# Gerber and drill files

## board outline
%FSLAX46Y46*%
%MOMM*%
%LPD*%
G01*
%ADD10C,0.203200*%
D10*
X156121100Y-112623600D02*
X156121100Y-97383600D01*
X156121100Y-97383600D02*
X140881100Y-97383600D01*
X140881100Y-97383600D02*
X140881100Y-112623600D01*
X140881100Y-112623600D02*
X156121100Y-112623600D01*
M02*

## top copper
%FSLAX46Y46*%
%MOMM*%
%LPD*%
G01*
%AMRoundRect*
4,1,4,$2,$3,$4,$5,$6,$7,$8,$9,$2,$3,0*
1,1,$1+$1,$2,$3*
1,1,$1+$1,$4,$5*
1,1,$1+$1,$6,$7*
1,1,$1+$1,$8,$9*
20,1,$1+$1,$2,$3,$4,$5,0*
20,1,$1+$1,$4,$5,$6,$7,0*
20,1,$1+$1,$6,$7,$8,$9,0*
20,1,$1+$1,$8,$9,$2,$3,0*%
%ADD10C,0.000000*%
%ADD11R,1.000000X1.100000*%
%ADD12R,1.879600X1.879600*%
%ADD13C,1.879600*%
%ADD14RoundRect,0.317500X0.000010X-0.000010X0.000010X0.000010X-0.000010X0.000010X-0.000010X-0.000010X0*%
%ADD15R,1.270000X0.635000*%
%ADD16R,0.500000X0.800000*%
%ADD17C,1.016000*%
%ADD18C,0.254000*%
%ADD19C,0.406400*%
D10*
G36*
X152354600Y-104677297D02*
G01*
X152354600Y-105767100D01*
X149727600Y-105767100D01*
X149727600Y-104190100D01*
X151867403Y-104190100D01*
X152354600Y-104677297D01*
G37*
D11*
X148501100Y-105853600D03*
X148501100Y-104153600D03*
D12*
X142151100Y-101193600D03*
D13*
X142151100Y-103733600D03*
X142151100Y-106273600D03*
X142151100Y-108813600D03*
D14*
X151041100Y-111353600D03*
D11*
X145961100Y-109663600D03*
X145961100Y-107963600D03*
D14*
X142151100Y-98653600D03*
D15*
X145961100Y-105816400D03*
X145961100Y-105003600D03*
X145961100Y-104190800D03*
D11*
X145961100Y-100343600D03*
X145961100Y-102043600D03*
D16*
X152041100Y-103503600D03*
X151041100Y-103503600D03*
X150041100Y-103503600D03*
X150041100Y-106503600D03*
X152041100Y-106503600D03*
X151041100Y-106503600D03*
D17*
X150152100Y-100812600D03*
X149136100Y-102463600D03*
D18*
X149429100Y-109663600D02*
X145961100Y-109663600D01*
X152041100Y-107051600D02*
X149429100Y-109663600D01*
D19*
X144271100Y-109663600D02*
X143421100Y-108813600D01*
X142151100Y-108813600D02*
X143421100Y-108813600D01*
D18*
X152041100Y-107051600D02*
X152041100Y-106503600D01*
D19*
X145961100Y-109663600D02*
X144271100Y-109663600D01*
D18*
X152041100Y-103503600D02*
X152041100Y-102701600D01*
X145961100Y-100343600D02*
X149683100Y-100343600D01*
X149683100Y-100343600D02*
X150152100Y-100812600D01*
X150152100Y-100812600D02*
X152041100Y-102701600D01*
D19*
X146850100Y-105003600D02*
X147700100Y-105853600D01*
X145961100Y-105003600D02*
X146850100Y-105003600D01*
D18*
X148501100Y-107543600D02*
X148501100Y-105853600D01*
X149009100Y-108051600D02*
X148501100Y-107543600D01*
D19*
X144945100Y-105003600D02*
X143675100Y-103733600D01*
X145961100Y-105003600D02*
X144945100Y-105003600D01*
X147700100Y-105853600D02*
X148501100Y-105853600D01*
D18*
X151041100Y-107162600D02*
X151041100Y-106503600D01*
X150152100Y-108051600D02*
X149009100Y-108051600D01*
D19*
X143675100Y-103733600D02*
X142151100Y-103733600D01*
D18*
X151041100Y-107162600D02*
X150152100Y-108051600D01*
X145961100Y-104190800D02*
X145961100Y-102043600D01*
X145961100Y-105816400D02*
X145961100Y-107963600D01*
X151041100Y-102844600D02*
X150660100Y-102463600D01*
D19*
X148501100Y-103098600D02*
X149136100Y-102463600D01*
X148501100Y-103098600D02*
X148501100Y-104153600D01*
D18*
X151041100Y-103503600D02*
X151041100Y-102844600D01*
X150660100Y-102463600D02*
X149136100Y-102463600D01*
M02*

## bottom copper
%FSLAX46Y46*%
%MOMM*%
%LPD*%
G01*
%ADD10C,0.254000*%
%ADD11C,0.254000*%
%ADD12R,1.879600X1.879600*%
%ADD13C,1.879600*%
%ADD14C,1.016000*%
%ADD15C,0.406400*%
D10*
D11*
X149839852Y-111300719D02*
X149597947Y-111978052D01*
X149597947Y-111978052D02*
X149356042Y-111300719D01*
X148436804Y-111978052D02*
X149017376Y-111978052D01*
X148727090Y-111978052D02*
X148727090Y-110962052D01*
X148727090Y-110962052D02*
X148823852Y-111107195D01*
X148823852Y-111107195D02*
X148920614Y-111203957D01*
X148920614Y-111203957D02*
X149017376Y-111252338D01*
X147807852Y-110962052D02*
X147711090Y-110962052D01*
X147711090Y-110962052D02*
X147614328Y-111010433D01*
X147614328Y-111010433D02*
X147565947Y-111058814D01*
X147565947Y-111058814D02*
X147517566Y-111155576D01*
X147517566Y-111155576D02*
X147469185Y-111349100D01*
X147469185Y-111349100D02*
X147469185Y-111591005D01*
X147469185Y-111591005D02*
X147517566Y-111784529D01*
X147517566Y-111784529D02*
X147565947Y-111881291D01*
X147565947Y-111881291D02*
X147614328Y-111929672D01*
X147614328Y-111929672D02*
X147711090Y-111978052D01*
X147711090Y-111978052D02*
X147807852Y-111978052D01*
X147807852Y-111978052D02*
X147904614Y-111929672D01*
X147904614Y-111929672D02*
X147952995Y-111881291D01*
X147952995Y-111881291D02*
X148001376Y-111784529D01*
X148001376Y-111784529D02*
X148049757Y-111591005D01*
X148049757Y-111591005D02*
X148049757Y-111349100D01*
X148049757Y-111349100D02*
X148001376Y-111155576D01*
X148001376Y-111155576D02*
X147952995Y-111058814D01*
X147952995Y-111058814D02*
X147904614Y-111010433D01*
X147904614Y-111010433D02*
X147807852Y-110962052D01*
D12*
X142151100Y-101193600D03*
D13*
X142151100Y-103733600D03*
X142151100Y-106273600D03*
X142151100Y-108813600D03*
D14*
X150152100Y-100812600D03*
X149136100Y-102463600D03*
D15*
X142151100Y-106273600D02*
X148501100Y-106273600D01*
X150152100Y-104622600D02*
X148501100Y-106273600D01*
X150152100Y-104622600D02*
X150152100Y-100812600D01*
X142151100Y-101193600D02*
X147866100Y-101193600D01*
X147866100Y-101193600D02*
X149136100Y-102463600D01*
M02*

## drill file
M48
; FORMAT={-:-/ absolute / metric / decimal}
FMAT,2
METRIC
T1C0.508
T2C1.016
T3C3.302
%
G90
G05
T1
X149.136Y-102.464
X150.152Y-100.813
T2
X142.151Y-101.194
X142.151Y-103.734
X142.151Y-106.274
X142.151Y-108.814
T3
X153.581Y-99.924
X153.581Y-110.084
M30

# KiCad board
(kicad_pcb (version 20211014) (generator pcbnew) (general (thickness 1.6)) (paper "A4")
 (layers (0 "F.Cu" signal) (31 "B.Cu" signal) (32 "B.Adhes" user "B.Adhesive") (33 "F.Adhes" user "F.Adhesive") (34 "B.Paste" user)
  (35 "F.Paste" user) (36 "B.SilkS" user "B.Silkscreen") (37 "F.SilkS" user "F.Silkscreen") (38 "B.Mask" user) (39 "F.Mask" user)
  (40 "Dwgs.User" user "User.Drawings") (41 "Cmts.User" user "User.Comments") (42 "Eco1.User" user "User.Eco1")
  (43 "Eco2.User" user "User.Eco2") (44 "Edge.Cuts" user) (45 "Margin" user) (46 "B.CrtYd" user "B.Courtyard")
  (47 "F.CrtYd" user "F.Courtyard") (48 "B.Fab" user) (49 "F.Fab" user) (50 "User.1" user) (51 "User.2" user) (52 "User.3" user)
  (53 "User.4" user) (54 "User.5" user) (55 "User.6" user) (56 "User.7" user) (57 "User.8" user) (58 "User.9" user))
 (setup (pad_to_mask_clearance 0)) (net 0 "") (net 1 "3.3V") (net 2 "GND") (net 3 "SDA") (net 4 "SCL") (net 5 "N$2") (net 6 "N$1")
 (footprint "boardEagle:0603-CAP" (layer "F.Cu") (at 148.5011 105.0036 90)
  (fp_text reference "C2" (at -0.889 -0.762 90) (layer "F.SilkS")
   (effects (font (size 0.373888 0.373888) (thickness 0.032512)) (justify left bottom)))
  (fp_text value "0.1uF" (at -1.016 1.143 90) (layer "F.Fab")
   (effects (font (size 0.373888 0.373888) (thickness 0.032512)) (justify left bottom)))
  (pad "1" smd rect (at -0.85 0 90) (size 1.1 1) (layers "F.Cu" "F.Paste" "F.Mask") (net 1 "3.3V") (solder_mask_margin 0.1016))
  (pad "2" smd rect (at 0.85 0 90) (size 1.1 1) (layers "F.Cu" "F.Paste" "F.Mask") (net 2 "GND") (solder_mask_margin 0.1016)))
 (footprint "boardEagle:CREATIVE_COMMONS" (layer "F.Cu") (at 128.1811 121.5136)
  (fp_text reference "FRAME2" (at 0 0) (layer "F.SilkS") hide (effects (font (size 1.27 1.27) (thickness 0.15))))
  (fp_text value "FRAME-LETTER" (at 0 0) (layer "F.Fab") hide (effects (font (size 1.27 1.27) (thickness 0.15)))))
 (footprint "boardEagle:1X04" (layer "F.Cu") (at 142.1511 101.1936 -90)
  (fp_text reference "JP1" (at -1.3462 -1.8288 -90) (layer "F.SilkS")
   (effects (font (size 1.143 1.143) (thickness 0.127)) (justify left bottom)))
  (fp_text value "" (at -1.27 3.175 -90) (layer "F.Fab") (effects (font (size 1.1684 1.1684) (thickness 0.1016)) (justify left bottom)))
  (pad "1" thru_hole rect (at 0 0) (size 1.8796 1.8796) (drill 1.016) (layers *.Cu *.Mask) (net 2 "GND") (solder_mask_margin 0.1016))
  (pad "2" thru_hole circle (at 2.54 0) (size 1.8796 1.8796) (drill 1.016) (layers *.Cu *.Mask) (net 1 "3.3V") (solder_mask_margin 0.1016))
  (pad "3" thru_hole circle (at 5.08 0) (size 1.8796 1.8796) (drill 1.016) (layers *.Cu *.Mask) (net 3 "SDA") (solder_mask_margin 0.1016))
  (pad "4" thru_hole circle (at 7.62 0) (size 1.8796 1.8796) (drill 1.016) (layers *.Cu *.Mask) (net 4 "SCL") (solder_mask_margin 0.1016)))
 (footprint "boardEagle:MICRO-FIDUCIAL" (layer "F.Cu") (at 151.0411 111.3536 90)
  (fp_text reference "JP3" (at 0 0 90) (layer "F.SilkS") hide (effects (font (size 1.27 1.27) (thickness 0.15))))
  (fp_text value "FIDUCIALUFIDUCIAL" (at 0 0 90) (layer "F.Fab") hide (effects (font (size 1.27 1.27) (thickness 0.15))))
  (pad "1" smd roundrect (at 0 0 90) (size 0.635 0.635) (layers "F.Cu" "F.Mask") (roundrect_rratio 0.5) (solder_mask_margin 0.1016)))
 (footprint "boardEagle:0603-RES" (layer "F.Cu") (at 145.9611 108.8136 90)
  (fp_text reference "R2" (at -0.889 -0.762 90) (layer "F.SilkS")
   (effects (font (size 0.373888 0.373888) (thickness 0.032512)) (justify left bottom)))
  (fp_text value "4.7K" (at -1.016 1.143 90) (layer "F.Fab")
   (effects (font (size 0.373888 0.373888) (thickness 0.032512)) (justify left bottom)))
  (pad "1" smd rect (at -0.85 0 90) (size 1.1 1) (layers "F.Cu" "F.Paste" "F.Mask") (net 4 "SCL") (solder_mask_margin 0.1016))
  (pad "2" smd rect (at 0.85 0 90) (size 1.1 1) (layers "F.Cu" "F.Paste" "F.Mask") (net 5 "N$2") (solder_mask_margin 0.1016)))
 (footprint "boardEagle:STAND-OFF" (layer "F.Cu") (at 153.5811 99.9236 90)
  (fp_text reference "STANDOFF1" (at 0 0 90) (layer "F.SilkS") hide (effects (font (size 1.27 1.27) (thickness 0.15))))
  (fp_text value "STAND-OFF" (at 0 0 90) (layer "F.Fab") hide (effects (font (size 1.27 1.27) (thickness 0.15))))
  (pad "" np_thru_hole circle (at 0 0 90) (size 3.302 3.302) (drill 3.302) (layers *.Cu *.Mask)))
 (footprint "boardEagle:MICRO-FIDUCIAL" (layer "F.Cu") (at 142.1511 98.6536 90)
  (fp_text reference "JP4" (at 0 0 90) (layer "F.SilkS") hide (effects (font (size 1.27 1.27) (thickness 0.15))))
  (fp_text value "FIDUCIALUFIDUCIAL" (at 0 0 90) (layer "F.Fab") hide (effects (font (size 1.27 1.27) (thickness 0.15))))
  (pad "1" smd roundrect (at 0 0 90) (size 0.635 0.635) (layers "F.Cu" "F.Mask") (roundrect_rratio 0.5) (solder_mask_margin 0.1016)))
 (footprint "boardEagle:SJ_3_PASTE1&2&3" (layer "F.Cu") (at 145.9611 105.0036 90)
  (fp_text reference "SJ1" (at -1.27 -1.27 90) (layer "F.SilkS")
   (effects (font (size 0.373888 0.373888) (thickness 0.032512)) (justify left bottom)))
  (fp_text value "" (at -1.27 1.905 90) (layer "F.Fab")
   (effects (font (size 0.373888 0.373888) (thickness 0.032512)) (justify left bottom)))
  (pad "1" smd rect (at -0.8128 0 90) (size 0.635 1.27) (layers "F.Cu" "F.Mask") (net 5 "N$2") (solder_mask_margin 0.1016))
  (pad "2" smd rect (at 0 0 90) (size 0.635 1.27) (layers "F.Cu" "F.Mask") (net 1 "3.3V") (solder_mask_margin 0.1016))
  (pad "3" smd rect (at 0.8128 0 90) (size 0.635 1.27) (layers "F.Cu" "F.Mask") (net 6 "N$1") (solder_mask_margin 0.1016)))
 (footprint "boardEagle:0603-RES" (layer "F.Cu") (at 145.9611 101.1936 -90)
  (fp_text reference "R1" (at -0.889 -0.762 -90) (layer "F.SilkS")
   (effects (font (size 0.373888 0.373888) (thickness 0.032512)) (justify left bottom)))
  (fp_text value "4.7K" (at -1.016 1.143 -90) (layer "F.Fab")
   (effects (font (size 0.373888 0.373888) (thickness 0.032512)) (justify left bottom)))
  (pad "1" smd rect (at -0.85 0 270) (size 1.1 1) (layers "F.Cu" "F.Paste" "F.Mask") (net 3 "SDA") (solder_mask_margin 0.1016))
  (pad "2" smd rect (at 0.85 0 270) (size 1.1 1) (layers "F.Cu" "F.Paste" "F.Mask") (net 6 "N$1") (solder_mask_margin 0.1016)))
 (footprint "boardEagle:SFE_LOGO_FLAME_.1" (layer "F.Cu") (at 152.9461 106.4006)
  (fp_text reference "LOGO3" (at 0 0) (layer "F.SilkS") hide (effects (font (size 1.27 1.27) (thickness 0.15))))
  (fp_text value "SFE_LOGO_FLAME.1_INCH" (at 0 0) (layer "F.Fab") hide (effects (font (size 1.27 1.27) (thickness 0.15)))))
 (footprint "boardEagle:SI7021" (layer "F.Cu") (at 151.0411 105.0036 90)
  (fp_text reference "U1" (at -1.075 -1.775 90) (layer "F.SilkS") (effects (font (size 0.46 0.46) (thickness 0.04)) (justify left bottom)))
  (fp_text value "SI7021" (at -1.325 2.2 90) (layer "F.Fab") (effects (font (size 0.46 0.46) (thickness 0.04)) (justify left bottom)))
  (fp_poly
   (pts (xy 0.8135 0.826303) (xy 0.326303 1.3135) (xy -0.7635 1.3135) (xy -0.7635 -1.3135) (xy 0.8135 -1.3135)) (layer "F.Cu") (width 0)
   (fill solid))
  (pad "DATA" smd rect (at 1.5 1) (size 0.5 0.8) (layers "F.Cu" "F.Paste" "F.Mask") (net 3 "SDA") (solder_mask_margin 0.1016))
  (pad "GND" smd rect (at 1.5 0) (size 0.5 0.8) (layers "F.Cu" "F.Paste" "F.Mask") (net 2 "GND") (solder_mask_margin 0.1016))
  (pad "NC@3" smd rect (at 1.5 -1) (size 0.5 0.8) (layers "F.Cu" "F.Paste" "F.Mask") (solder_mask_margin 0.1016))
  (pad "NC@4" smd rect (at -1.5 -1) (size 0.5 0.8) (layers "F.Cu" "F.Paste" "F.Mask") (solder_mask_margin 0.1016))
  (pad "SCK" smd rect (at -1.5 1) (size 0.5 0.8) (layers "F.Cu" "F.Paste" "F.Mask") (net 4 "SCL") (solder_mask_margin 0.1016))
  (pad "VDD" smd rect (at -1.5 0) (size 0.5 0.8) (layers "F.Cu" "F.Paste" "F.Mask") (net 1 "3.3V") (solder_mask_margin 0.1016)))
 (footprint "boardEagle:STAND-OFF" (layer "F.Cu") (at 153.5811 110.0836 90)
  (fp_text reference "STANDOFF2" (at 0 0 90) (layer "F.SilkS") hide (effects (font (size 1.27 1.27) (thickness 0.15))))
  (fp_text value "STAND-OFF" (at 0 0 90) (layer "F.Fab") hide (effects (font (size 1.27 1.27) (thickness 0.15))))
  (pad "" np_thru_hole circle (at 0 0 90) (size 3.302 3.302) (drill 3.302) (layers *.Cu *.Mask)))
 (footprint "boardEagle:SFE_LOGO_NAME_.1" (layer "B.Cu") (at 149.7711 98.6536 -90)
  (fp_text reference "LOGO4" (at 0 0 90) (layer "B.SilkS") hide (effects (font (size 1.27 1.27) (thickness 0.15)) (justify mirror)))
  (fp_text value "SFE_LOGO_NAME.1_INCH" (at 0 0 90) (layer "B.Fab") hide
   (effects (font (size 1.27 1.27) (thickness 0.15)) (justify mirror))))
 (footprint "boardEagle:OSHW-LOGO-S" (layer "B.Cu") (at 153.5811 105.1306 -90)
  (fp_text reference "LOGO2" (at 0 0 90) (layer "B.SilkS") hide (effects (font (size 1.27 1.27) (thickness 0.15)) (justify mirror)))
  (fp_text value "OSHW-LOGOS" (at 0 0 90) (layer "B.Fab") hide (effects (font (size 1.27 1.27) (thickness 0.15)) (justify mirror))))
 (gr_line (start 156.1211 112.6236) (end 156.1211 97.3836) (layer "Edge.Cuts") (width 0.2032))
 (gr_line (start 156.1211 97.3836) (end 140.8811 97.3836) (layer "Edge.Cuts") (width 0.2032))
 (gr_line (start 140.8811 97.3836) (end 140.8811 112.6236) (layer "Edge.Cuts") (width 0.2032))
 (gr_line (start 140.8811 112.6236) (end 156.1211 112.6236) (layer "Edge.Cuts") (width 0.2032))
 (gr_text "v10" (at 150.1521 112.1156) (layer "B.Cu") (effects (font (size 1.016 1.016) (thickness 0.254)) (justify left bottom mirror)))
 (segment (start 149.4291 109.6636) (end 145.9611 109.6636) (width 0.254) (layer "F.Cu") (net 4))
 (segment (start 152.0411 107.0516) (end 149.4291 109.6636) (width 0.254) (layer "F.Cu") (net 4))
 (segment (start 144.2711 109.6636) (end 143.4211 108.8136) (width 0.4064) (layer "F.Cu") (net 4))
 (segment (start 142.1511 108.8136) (end 143.4211 108.8136) (width 0.4064) (layer "F.Cu") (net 4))
 (segment (start 152.0411 107.0516) (end 152.0411 106.5036) (width 0.254) (layer "F.Cu") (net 4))
 (segment (start 145.9611 109.6636) (end 144.2711 109.6636) (width 0.4064) (layer "F.Cu") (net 4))
 (segment (start 152.0411 103.5036) (end 152.0411 102.7016) (width 0.254) (layer "F.Cu") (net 3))
 (segment (start 145.9611 100.3436) (end 149.6831 100.3436) (width 0.254) (layer "F.Cu") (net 3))
 (segment (start 149.6831 100.3436) (end 150.1521 100.8126) (width 0.254) (layer "F.Cu") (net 3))
 (segment (start 150.1521 100.8126) (end 152.0411 102.7016) (width 0.254) (layer "F.Cu") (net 3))
 (via (at 150.1521 100.8126) (size 1.016) (drill 0.508) (layers "F.Cu" "B.Cu") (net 3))
 (segment (start 142.1511 106.2736) (end 148.5011 106.2736) (width 0.4064) (layer "B.Cu") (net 3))
 (segment (start 150.1521 104.6226) (end 148.5011 106.2736) (width 0.4064) (layer "B.Cu") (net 3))
 (segment (start 150.1521 104.6226) (end 150.1521 100.8126) (width 0.4064) (layer "B.Cu") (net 3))
 (segment (start 146.8501 105.0036) (end 147.7001 105.8536) (width 0.4064) (layer "F.Cu") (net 1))
 (segment (start 145.9611 105.0036) (end 146.8501 105.0036) (width 0.4064) (layer "F.Cu") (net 1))
 (segment (start 148.5011 107.5436) (end 148.5011 105.8536) (width 0.254) (layer "F.Cu") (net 1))
 (segment (start 149.0091 108.0516) (end 148.5011 107.5436) (width 0.254) (layer "F.Cu") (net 1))
 (segment (start 144.9451 105.0036) (end 143.6751 103.7336) (width 0.4064) (layer "F.Cu") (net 1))
 (segment (start 145.9611 105.0036) (end 144.9451 105.0036) (width 0.4064) (layer "F.Cu") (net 1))
 (segment (start 147.7001 105.8536) (end 148.5011 105.8536) (width 0.4064) (layer "F.Cu") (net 1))
 (segment (start 151.0411 107.1626) (end 151.0411 106.5036) (width 0.254) (layer "F.Cu") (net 1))
 (segment (start 150.1521 108.0516) (end 149.0091 108.0516) (width 0.254) (layer "F.Cu") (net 1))
 (segment (start 143.6751 103.7336) (end 142.1511 103.7336) (width 0.4064) (layer "F.Cu") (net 1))
 (segment (start 151.0411 107.1626) (end 150.1521 108.0516) (width 0.254) (layer "F.Cu") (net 1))
 (segment (start 145.9611 104.1908) (end 145.9611 102.0436) (width 0.254) (layer "F.Cu") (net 6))
 (segment (start 145.9611 105.8164) (end 145.9611 107.9636) (width 0.254) (layer "F.Cu") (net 5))
 (segment (start 151.0411 102.8446) (end 150.6601 102.4636) (width 0.254) (layer "F.Cu") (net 2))
 (segment (start 148.5011 103.0986) (end 149.1361 102.4636) (width 0.4064) (layer "F.Cu") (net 2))
 (segment (start 148.5011 103.0986) (end 148.5011 104.1536) (width 0.4064) (layer "F.Cu") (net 2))
 (segment (start 151.0411 103.5036) (end 151.0411 102.8446) (width 0.254) (layer "F.Cu") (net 2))
 (segment (start 150.6601 102.4636) (end 149.1361 102.4636) (width 0.254) (layer "F.Cu") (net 2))
 (via (at 149.1361 102.4636) (size 1.016) (drill 0.508) (layers "F.Cu" "B.Cu") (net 2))
 (segment (start 142.1511 101.1936) (end 147.8661 101.1936) (width 0.4064) (layer "B.Cu") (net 2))
 (segment (start 147.8661 101.1936) (end 149.1361 102.4636) (width 0.4064) (layer "B.Cu") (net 2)))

